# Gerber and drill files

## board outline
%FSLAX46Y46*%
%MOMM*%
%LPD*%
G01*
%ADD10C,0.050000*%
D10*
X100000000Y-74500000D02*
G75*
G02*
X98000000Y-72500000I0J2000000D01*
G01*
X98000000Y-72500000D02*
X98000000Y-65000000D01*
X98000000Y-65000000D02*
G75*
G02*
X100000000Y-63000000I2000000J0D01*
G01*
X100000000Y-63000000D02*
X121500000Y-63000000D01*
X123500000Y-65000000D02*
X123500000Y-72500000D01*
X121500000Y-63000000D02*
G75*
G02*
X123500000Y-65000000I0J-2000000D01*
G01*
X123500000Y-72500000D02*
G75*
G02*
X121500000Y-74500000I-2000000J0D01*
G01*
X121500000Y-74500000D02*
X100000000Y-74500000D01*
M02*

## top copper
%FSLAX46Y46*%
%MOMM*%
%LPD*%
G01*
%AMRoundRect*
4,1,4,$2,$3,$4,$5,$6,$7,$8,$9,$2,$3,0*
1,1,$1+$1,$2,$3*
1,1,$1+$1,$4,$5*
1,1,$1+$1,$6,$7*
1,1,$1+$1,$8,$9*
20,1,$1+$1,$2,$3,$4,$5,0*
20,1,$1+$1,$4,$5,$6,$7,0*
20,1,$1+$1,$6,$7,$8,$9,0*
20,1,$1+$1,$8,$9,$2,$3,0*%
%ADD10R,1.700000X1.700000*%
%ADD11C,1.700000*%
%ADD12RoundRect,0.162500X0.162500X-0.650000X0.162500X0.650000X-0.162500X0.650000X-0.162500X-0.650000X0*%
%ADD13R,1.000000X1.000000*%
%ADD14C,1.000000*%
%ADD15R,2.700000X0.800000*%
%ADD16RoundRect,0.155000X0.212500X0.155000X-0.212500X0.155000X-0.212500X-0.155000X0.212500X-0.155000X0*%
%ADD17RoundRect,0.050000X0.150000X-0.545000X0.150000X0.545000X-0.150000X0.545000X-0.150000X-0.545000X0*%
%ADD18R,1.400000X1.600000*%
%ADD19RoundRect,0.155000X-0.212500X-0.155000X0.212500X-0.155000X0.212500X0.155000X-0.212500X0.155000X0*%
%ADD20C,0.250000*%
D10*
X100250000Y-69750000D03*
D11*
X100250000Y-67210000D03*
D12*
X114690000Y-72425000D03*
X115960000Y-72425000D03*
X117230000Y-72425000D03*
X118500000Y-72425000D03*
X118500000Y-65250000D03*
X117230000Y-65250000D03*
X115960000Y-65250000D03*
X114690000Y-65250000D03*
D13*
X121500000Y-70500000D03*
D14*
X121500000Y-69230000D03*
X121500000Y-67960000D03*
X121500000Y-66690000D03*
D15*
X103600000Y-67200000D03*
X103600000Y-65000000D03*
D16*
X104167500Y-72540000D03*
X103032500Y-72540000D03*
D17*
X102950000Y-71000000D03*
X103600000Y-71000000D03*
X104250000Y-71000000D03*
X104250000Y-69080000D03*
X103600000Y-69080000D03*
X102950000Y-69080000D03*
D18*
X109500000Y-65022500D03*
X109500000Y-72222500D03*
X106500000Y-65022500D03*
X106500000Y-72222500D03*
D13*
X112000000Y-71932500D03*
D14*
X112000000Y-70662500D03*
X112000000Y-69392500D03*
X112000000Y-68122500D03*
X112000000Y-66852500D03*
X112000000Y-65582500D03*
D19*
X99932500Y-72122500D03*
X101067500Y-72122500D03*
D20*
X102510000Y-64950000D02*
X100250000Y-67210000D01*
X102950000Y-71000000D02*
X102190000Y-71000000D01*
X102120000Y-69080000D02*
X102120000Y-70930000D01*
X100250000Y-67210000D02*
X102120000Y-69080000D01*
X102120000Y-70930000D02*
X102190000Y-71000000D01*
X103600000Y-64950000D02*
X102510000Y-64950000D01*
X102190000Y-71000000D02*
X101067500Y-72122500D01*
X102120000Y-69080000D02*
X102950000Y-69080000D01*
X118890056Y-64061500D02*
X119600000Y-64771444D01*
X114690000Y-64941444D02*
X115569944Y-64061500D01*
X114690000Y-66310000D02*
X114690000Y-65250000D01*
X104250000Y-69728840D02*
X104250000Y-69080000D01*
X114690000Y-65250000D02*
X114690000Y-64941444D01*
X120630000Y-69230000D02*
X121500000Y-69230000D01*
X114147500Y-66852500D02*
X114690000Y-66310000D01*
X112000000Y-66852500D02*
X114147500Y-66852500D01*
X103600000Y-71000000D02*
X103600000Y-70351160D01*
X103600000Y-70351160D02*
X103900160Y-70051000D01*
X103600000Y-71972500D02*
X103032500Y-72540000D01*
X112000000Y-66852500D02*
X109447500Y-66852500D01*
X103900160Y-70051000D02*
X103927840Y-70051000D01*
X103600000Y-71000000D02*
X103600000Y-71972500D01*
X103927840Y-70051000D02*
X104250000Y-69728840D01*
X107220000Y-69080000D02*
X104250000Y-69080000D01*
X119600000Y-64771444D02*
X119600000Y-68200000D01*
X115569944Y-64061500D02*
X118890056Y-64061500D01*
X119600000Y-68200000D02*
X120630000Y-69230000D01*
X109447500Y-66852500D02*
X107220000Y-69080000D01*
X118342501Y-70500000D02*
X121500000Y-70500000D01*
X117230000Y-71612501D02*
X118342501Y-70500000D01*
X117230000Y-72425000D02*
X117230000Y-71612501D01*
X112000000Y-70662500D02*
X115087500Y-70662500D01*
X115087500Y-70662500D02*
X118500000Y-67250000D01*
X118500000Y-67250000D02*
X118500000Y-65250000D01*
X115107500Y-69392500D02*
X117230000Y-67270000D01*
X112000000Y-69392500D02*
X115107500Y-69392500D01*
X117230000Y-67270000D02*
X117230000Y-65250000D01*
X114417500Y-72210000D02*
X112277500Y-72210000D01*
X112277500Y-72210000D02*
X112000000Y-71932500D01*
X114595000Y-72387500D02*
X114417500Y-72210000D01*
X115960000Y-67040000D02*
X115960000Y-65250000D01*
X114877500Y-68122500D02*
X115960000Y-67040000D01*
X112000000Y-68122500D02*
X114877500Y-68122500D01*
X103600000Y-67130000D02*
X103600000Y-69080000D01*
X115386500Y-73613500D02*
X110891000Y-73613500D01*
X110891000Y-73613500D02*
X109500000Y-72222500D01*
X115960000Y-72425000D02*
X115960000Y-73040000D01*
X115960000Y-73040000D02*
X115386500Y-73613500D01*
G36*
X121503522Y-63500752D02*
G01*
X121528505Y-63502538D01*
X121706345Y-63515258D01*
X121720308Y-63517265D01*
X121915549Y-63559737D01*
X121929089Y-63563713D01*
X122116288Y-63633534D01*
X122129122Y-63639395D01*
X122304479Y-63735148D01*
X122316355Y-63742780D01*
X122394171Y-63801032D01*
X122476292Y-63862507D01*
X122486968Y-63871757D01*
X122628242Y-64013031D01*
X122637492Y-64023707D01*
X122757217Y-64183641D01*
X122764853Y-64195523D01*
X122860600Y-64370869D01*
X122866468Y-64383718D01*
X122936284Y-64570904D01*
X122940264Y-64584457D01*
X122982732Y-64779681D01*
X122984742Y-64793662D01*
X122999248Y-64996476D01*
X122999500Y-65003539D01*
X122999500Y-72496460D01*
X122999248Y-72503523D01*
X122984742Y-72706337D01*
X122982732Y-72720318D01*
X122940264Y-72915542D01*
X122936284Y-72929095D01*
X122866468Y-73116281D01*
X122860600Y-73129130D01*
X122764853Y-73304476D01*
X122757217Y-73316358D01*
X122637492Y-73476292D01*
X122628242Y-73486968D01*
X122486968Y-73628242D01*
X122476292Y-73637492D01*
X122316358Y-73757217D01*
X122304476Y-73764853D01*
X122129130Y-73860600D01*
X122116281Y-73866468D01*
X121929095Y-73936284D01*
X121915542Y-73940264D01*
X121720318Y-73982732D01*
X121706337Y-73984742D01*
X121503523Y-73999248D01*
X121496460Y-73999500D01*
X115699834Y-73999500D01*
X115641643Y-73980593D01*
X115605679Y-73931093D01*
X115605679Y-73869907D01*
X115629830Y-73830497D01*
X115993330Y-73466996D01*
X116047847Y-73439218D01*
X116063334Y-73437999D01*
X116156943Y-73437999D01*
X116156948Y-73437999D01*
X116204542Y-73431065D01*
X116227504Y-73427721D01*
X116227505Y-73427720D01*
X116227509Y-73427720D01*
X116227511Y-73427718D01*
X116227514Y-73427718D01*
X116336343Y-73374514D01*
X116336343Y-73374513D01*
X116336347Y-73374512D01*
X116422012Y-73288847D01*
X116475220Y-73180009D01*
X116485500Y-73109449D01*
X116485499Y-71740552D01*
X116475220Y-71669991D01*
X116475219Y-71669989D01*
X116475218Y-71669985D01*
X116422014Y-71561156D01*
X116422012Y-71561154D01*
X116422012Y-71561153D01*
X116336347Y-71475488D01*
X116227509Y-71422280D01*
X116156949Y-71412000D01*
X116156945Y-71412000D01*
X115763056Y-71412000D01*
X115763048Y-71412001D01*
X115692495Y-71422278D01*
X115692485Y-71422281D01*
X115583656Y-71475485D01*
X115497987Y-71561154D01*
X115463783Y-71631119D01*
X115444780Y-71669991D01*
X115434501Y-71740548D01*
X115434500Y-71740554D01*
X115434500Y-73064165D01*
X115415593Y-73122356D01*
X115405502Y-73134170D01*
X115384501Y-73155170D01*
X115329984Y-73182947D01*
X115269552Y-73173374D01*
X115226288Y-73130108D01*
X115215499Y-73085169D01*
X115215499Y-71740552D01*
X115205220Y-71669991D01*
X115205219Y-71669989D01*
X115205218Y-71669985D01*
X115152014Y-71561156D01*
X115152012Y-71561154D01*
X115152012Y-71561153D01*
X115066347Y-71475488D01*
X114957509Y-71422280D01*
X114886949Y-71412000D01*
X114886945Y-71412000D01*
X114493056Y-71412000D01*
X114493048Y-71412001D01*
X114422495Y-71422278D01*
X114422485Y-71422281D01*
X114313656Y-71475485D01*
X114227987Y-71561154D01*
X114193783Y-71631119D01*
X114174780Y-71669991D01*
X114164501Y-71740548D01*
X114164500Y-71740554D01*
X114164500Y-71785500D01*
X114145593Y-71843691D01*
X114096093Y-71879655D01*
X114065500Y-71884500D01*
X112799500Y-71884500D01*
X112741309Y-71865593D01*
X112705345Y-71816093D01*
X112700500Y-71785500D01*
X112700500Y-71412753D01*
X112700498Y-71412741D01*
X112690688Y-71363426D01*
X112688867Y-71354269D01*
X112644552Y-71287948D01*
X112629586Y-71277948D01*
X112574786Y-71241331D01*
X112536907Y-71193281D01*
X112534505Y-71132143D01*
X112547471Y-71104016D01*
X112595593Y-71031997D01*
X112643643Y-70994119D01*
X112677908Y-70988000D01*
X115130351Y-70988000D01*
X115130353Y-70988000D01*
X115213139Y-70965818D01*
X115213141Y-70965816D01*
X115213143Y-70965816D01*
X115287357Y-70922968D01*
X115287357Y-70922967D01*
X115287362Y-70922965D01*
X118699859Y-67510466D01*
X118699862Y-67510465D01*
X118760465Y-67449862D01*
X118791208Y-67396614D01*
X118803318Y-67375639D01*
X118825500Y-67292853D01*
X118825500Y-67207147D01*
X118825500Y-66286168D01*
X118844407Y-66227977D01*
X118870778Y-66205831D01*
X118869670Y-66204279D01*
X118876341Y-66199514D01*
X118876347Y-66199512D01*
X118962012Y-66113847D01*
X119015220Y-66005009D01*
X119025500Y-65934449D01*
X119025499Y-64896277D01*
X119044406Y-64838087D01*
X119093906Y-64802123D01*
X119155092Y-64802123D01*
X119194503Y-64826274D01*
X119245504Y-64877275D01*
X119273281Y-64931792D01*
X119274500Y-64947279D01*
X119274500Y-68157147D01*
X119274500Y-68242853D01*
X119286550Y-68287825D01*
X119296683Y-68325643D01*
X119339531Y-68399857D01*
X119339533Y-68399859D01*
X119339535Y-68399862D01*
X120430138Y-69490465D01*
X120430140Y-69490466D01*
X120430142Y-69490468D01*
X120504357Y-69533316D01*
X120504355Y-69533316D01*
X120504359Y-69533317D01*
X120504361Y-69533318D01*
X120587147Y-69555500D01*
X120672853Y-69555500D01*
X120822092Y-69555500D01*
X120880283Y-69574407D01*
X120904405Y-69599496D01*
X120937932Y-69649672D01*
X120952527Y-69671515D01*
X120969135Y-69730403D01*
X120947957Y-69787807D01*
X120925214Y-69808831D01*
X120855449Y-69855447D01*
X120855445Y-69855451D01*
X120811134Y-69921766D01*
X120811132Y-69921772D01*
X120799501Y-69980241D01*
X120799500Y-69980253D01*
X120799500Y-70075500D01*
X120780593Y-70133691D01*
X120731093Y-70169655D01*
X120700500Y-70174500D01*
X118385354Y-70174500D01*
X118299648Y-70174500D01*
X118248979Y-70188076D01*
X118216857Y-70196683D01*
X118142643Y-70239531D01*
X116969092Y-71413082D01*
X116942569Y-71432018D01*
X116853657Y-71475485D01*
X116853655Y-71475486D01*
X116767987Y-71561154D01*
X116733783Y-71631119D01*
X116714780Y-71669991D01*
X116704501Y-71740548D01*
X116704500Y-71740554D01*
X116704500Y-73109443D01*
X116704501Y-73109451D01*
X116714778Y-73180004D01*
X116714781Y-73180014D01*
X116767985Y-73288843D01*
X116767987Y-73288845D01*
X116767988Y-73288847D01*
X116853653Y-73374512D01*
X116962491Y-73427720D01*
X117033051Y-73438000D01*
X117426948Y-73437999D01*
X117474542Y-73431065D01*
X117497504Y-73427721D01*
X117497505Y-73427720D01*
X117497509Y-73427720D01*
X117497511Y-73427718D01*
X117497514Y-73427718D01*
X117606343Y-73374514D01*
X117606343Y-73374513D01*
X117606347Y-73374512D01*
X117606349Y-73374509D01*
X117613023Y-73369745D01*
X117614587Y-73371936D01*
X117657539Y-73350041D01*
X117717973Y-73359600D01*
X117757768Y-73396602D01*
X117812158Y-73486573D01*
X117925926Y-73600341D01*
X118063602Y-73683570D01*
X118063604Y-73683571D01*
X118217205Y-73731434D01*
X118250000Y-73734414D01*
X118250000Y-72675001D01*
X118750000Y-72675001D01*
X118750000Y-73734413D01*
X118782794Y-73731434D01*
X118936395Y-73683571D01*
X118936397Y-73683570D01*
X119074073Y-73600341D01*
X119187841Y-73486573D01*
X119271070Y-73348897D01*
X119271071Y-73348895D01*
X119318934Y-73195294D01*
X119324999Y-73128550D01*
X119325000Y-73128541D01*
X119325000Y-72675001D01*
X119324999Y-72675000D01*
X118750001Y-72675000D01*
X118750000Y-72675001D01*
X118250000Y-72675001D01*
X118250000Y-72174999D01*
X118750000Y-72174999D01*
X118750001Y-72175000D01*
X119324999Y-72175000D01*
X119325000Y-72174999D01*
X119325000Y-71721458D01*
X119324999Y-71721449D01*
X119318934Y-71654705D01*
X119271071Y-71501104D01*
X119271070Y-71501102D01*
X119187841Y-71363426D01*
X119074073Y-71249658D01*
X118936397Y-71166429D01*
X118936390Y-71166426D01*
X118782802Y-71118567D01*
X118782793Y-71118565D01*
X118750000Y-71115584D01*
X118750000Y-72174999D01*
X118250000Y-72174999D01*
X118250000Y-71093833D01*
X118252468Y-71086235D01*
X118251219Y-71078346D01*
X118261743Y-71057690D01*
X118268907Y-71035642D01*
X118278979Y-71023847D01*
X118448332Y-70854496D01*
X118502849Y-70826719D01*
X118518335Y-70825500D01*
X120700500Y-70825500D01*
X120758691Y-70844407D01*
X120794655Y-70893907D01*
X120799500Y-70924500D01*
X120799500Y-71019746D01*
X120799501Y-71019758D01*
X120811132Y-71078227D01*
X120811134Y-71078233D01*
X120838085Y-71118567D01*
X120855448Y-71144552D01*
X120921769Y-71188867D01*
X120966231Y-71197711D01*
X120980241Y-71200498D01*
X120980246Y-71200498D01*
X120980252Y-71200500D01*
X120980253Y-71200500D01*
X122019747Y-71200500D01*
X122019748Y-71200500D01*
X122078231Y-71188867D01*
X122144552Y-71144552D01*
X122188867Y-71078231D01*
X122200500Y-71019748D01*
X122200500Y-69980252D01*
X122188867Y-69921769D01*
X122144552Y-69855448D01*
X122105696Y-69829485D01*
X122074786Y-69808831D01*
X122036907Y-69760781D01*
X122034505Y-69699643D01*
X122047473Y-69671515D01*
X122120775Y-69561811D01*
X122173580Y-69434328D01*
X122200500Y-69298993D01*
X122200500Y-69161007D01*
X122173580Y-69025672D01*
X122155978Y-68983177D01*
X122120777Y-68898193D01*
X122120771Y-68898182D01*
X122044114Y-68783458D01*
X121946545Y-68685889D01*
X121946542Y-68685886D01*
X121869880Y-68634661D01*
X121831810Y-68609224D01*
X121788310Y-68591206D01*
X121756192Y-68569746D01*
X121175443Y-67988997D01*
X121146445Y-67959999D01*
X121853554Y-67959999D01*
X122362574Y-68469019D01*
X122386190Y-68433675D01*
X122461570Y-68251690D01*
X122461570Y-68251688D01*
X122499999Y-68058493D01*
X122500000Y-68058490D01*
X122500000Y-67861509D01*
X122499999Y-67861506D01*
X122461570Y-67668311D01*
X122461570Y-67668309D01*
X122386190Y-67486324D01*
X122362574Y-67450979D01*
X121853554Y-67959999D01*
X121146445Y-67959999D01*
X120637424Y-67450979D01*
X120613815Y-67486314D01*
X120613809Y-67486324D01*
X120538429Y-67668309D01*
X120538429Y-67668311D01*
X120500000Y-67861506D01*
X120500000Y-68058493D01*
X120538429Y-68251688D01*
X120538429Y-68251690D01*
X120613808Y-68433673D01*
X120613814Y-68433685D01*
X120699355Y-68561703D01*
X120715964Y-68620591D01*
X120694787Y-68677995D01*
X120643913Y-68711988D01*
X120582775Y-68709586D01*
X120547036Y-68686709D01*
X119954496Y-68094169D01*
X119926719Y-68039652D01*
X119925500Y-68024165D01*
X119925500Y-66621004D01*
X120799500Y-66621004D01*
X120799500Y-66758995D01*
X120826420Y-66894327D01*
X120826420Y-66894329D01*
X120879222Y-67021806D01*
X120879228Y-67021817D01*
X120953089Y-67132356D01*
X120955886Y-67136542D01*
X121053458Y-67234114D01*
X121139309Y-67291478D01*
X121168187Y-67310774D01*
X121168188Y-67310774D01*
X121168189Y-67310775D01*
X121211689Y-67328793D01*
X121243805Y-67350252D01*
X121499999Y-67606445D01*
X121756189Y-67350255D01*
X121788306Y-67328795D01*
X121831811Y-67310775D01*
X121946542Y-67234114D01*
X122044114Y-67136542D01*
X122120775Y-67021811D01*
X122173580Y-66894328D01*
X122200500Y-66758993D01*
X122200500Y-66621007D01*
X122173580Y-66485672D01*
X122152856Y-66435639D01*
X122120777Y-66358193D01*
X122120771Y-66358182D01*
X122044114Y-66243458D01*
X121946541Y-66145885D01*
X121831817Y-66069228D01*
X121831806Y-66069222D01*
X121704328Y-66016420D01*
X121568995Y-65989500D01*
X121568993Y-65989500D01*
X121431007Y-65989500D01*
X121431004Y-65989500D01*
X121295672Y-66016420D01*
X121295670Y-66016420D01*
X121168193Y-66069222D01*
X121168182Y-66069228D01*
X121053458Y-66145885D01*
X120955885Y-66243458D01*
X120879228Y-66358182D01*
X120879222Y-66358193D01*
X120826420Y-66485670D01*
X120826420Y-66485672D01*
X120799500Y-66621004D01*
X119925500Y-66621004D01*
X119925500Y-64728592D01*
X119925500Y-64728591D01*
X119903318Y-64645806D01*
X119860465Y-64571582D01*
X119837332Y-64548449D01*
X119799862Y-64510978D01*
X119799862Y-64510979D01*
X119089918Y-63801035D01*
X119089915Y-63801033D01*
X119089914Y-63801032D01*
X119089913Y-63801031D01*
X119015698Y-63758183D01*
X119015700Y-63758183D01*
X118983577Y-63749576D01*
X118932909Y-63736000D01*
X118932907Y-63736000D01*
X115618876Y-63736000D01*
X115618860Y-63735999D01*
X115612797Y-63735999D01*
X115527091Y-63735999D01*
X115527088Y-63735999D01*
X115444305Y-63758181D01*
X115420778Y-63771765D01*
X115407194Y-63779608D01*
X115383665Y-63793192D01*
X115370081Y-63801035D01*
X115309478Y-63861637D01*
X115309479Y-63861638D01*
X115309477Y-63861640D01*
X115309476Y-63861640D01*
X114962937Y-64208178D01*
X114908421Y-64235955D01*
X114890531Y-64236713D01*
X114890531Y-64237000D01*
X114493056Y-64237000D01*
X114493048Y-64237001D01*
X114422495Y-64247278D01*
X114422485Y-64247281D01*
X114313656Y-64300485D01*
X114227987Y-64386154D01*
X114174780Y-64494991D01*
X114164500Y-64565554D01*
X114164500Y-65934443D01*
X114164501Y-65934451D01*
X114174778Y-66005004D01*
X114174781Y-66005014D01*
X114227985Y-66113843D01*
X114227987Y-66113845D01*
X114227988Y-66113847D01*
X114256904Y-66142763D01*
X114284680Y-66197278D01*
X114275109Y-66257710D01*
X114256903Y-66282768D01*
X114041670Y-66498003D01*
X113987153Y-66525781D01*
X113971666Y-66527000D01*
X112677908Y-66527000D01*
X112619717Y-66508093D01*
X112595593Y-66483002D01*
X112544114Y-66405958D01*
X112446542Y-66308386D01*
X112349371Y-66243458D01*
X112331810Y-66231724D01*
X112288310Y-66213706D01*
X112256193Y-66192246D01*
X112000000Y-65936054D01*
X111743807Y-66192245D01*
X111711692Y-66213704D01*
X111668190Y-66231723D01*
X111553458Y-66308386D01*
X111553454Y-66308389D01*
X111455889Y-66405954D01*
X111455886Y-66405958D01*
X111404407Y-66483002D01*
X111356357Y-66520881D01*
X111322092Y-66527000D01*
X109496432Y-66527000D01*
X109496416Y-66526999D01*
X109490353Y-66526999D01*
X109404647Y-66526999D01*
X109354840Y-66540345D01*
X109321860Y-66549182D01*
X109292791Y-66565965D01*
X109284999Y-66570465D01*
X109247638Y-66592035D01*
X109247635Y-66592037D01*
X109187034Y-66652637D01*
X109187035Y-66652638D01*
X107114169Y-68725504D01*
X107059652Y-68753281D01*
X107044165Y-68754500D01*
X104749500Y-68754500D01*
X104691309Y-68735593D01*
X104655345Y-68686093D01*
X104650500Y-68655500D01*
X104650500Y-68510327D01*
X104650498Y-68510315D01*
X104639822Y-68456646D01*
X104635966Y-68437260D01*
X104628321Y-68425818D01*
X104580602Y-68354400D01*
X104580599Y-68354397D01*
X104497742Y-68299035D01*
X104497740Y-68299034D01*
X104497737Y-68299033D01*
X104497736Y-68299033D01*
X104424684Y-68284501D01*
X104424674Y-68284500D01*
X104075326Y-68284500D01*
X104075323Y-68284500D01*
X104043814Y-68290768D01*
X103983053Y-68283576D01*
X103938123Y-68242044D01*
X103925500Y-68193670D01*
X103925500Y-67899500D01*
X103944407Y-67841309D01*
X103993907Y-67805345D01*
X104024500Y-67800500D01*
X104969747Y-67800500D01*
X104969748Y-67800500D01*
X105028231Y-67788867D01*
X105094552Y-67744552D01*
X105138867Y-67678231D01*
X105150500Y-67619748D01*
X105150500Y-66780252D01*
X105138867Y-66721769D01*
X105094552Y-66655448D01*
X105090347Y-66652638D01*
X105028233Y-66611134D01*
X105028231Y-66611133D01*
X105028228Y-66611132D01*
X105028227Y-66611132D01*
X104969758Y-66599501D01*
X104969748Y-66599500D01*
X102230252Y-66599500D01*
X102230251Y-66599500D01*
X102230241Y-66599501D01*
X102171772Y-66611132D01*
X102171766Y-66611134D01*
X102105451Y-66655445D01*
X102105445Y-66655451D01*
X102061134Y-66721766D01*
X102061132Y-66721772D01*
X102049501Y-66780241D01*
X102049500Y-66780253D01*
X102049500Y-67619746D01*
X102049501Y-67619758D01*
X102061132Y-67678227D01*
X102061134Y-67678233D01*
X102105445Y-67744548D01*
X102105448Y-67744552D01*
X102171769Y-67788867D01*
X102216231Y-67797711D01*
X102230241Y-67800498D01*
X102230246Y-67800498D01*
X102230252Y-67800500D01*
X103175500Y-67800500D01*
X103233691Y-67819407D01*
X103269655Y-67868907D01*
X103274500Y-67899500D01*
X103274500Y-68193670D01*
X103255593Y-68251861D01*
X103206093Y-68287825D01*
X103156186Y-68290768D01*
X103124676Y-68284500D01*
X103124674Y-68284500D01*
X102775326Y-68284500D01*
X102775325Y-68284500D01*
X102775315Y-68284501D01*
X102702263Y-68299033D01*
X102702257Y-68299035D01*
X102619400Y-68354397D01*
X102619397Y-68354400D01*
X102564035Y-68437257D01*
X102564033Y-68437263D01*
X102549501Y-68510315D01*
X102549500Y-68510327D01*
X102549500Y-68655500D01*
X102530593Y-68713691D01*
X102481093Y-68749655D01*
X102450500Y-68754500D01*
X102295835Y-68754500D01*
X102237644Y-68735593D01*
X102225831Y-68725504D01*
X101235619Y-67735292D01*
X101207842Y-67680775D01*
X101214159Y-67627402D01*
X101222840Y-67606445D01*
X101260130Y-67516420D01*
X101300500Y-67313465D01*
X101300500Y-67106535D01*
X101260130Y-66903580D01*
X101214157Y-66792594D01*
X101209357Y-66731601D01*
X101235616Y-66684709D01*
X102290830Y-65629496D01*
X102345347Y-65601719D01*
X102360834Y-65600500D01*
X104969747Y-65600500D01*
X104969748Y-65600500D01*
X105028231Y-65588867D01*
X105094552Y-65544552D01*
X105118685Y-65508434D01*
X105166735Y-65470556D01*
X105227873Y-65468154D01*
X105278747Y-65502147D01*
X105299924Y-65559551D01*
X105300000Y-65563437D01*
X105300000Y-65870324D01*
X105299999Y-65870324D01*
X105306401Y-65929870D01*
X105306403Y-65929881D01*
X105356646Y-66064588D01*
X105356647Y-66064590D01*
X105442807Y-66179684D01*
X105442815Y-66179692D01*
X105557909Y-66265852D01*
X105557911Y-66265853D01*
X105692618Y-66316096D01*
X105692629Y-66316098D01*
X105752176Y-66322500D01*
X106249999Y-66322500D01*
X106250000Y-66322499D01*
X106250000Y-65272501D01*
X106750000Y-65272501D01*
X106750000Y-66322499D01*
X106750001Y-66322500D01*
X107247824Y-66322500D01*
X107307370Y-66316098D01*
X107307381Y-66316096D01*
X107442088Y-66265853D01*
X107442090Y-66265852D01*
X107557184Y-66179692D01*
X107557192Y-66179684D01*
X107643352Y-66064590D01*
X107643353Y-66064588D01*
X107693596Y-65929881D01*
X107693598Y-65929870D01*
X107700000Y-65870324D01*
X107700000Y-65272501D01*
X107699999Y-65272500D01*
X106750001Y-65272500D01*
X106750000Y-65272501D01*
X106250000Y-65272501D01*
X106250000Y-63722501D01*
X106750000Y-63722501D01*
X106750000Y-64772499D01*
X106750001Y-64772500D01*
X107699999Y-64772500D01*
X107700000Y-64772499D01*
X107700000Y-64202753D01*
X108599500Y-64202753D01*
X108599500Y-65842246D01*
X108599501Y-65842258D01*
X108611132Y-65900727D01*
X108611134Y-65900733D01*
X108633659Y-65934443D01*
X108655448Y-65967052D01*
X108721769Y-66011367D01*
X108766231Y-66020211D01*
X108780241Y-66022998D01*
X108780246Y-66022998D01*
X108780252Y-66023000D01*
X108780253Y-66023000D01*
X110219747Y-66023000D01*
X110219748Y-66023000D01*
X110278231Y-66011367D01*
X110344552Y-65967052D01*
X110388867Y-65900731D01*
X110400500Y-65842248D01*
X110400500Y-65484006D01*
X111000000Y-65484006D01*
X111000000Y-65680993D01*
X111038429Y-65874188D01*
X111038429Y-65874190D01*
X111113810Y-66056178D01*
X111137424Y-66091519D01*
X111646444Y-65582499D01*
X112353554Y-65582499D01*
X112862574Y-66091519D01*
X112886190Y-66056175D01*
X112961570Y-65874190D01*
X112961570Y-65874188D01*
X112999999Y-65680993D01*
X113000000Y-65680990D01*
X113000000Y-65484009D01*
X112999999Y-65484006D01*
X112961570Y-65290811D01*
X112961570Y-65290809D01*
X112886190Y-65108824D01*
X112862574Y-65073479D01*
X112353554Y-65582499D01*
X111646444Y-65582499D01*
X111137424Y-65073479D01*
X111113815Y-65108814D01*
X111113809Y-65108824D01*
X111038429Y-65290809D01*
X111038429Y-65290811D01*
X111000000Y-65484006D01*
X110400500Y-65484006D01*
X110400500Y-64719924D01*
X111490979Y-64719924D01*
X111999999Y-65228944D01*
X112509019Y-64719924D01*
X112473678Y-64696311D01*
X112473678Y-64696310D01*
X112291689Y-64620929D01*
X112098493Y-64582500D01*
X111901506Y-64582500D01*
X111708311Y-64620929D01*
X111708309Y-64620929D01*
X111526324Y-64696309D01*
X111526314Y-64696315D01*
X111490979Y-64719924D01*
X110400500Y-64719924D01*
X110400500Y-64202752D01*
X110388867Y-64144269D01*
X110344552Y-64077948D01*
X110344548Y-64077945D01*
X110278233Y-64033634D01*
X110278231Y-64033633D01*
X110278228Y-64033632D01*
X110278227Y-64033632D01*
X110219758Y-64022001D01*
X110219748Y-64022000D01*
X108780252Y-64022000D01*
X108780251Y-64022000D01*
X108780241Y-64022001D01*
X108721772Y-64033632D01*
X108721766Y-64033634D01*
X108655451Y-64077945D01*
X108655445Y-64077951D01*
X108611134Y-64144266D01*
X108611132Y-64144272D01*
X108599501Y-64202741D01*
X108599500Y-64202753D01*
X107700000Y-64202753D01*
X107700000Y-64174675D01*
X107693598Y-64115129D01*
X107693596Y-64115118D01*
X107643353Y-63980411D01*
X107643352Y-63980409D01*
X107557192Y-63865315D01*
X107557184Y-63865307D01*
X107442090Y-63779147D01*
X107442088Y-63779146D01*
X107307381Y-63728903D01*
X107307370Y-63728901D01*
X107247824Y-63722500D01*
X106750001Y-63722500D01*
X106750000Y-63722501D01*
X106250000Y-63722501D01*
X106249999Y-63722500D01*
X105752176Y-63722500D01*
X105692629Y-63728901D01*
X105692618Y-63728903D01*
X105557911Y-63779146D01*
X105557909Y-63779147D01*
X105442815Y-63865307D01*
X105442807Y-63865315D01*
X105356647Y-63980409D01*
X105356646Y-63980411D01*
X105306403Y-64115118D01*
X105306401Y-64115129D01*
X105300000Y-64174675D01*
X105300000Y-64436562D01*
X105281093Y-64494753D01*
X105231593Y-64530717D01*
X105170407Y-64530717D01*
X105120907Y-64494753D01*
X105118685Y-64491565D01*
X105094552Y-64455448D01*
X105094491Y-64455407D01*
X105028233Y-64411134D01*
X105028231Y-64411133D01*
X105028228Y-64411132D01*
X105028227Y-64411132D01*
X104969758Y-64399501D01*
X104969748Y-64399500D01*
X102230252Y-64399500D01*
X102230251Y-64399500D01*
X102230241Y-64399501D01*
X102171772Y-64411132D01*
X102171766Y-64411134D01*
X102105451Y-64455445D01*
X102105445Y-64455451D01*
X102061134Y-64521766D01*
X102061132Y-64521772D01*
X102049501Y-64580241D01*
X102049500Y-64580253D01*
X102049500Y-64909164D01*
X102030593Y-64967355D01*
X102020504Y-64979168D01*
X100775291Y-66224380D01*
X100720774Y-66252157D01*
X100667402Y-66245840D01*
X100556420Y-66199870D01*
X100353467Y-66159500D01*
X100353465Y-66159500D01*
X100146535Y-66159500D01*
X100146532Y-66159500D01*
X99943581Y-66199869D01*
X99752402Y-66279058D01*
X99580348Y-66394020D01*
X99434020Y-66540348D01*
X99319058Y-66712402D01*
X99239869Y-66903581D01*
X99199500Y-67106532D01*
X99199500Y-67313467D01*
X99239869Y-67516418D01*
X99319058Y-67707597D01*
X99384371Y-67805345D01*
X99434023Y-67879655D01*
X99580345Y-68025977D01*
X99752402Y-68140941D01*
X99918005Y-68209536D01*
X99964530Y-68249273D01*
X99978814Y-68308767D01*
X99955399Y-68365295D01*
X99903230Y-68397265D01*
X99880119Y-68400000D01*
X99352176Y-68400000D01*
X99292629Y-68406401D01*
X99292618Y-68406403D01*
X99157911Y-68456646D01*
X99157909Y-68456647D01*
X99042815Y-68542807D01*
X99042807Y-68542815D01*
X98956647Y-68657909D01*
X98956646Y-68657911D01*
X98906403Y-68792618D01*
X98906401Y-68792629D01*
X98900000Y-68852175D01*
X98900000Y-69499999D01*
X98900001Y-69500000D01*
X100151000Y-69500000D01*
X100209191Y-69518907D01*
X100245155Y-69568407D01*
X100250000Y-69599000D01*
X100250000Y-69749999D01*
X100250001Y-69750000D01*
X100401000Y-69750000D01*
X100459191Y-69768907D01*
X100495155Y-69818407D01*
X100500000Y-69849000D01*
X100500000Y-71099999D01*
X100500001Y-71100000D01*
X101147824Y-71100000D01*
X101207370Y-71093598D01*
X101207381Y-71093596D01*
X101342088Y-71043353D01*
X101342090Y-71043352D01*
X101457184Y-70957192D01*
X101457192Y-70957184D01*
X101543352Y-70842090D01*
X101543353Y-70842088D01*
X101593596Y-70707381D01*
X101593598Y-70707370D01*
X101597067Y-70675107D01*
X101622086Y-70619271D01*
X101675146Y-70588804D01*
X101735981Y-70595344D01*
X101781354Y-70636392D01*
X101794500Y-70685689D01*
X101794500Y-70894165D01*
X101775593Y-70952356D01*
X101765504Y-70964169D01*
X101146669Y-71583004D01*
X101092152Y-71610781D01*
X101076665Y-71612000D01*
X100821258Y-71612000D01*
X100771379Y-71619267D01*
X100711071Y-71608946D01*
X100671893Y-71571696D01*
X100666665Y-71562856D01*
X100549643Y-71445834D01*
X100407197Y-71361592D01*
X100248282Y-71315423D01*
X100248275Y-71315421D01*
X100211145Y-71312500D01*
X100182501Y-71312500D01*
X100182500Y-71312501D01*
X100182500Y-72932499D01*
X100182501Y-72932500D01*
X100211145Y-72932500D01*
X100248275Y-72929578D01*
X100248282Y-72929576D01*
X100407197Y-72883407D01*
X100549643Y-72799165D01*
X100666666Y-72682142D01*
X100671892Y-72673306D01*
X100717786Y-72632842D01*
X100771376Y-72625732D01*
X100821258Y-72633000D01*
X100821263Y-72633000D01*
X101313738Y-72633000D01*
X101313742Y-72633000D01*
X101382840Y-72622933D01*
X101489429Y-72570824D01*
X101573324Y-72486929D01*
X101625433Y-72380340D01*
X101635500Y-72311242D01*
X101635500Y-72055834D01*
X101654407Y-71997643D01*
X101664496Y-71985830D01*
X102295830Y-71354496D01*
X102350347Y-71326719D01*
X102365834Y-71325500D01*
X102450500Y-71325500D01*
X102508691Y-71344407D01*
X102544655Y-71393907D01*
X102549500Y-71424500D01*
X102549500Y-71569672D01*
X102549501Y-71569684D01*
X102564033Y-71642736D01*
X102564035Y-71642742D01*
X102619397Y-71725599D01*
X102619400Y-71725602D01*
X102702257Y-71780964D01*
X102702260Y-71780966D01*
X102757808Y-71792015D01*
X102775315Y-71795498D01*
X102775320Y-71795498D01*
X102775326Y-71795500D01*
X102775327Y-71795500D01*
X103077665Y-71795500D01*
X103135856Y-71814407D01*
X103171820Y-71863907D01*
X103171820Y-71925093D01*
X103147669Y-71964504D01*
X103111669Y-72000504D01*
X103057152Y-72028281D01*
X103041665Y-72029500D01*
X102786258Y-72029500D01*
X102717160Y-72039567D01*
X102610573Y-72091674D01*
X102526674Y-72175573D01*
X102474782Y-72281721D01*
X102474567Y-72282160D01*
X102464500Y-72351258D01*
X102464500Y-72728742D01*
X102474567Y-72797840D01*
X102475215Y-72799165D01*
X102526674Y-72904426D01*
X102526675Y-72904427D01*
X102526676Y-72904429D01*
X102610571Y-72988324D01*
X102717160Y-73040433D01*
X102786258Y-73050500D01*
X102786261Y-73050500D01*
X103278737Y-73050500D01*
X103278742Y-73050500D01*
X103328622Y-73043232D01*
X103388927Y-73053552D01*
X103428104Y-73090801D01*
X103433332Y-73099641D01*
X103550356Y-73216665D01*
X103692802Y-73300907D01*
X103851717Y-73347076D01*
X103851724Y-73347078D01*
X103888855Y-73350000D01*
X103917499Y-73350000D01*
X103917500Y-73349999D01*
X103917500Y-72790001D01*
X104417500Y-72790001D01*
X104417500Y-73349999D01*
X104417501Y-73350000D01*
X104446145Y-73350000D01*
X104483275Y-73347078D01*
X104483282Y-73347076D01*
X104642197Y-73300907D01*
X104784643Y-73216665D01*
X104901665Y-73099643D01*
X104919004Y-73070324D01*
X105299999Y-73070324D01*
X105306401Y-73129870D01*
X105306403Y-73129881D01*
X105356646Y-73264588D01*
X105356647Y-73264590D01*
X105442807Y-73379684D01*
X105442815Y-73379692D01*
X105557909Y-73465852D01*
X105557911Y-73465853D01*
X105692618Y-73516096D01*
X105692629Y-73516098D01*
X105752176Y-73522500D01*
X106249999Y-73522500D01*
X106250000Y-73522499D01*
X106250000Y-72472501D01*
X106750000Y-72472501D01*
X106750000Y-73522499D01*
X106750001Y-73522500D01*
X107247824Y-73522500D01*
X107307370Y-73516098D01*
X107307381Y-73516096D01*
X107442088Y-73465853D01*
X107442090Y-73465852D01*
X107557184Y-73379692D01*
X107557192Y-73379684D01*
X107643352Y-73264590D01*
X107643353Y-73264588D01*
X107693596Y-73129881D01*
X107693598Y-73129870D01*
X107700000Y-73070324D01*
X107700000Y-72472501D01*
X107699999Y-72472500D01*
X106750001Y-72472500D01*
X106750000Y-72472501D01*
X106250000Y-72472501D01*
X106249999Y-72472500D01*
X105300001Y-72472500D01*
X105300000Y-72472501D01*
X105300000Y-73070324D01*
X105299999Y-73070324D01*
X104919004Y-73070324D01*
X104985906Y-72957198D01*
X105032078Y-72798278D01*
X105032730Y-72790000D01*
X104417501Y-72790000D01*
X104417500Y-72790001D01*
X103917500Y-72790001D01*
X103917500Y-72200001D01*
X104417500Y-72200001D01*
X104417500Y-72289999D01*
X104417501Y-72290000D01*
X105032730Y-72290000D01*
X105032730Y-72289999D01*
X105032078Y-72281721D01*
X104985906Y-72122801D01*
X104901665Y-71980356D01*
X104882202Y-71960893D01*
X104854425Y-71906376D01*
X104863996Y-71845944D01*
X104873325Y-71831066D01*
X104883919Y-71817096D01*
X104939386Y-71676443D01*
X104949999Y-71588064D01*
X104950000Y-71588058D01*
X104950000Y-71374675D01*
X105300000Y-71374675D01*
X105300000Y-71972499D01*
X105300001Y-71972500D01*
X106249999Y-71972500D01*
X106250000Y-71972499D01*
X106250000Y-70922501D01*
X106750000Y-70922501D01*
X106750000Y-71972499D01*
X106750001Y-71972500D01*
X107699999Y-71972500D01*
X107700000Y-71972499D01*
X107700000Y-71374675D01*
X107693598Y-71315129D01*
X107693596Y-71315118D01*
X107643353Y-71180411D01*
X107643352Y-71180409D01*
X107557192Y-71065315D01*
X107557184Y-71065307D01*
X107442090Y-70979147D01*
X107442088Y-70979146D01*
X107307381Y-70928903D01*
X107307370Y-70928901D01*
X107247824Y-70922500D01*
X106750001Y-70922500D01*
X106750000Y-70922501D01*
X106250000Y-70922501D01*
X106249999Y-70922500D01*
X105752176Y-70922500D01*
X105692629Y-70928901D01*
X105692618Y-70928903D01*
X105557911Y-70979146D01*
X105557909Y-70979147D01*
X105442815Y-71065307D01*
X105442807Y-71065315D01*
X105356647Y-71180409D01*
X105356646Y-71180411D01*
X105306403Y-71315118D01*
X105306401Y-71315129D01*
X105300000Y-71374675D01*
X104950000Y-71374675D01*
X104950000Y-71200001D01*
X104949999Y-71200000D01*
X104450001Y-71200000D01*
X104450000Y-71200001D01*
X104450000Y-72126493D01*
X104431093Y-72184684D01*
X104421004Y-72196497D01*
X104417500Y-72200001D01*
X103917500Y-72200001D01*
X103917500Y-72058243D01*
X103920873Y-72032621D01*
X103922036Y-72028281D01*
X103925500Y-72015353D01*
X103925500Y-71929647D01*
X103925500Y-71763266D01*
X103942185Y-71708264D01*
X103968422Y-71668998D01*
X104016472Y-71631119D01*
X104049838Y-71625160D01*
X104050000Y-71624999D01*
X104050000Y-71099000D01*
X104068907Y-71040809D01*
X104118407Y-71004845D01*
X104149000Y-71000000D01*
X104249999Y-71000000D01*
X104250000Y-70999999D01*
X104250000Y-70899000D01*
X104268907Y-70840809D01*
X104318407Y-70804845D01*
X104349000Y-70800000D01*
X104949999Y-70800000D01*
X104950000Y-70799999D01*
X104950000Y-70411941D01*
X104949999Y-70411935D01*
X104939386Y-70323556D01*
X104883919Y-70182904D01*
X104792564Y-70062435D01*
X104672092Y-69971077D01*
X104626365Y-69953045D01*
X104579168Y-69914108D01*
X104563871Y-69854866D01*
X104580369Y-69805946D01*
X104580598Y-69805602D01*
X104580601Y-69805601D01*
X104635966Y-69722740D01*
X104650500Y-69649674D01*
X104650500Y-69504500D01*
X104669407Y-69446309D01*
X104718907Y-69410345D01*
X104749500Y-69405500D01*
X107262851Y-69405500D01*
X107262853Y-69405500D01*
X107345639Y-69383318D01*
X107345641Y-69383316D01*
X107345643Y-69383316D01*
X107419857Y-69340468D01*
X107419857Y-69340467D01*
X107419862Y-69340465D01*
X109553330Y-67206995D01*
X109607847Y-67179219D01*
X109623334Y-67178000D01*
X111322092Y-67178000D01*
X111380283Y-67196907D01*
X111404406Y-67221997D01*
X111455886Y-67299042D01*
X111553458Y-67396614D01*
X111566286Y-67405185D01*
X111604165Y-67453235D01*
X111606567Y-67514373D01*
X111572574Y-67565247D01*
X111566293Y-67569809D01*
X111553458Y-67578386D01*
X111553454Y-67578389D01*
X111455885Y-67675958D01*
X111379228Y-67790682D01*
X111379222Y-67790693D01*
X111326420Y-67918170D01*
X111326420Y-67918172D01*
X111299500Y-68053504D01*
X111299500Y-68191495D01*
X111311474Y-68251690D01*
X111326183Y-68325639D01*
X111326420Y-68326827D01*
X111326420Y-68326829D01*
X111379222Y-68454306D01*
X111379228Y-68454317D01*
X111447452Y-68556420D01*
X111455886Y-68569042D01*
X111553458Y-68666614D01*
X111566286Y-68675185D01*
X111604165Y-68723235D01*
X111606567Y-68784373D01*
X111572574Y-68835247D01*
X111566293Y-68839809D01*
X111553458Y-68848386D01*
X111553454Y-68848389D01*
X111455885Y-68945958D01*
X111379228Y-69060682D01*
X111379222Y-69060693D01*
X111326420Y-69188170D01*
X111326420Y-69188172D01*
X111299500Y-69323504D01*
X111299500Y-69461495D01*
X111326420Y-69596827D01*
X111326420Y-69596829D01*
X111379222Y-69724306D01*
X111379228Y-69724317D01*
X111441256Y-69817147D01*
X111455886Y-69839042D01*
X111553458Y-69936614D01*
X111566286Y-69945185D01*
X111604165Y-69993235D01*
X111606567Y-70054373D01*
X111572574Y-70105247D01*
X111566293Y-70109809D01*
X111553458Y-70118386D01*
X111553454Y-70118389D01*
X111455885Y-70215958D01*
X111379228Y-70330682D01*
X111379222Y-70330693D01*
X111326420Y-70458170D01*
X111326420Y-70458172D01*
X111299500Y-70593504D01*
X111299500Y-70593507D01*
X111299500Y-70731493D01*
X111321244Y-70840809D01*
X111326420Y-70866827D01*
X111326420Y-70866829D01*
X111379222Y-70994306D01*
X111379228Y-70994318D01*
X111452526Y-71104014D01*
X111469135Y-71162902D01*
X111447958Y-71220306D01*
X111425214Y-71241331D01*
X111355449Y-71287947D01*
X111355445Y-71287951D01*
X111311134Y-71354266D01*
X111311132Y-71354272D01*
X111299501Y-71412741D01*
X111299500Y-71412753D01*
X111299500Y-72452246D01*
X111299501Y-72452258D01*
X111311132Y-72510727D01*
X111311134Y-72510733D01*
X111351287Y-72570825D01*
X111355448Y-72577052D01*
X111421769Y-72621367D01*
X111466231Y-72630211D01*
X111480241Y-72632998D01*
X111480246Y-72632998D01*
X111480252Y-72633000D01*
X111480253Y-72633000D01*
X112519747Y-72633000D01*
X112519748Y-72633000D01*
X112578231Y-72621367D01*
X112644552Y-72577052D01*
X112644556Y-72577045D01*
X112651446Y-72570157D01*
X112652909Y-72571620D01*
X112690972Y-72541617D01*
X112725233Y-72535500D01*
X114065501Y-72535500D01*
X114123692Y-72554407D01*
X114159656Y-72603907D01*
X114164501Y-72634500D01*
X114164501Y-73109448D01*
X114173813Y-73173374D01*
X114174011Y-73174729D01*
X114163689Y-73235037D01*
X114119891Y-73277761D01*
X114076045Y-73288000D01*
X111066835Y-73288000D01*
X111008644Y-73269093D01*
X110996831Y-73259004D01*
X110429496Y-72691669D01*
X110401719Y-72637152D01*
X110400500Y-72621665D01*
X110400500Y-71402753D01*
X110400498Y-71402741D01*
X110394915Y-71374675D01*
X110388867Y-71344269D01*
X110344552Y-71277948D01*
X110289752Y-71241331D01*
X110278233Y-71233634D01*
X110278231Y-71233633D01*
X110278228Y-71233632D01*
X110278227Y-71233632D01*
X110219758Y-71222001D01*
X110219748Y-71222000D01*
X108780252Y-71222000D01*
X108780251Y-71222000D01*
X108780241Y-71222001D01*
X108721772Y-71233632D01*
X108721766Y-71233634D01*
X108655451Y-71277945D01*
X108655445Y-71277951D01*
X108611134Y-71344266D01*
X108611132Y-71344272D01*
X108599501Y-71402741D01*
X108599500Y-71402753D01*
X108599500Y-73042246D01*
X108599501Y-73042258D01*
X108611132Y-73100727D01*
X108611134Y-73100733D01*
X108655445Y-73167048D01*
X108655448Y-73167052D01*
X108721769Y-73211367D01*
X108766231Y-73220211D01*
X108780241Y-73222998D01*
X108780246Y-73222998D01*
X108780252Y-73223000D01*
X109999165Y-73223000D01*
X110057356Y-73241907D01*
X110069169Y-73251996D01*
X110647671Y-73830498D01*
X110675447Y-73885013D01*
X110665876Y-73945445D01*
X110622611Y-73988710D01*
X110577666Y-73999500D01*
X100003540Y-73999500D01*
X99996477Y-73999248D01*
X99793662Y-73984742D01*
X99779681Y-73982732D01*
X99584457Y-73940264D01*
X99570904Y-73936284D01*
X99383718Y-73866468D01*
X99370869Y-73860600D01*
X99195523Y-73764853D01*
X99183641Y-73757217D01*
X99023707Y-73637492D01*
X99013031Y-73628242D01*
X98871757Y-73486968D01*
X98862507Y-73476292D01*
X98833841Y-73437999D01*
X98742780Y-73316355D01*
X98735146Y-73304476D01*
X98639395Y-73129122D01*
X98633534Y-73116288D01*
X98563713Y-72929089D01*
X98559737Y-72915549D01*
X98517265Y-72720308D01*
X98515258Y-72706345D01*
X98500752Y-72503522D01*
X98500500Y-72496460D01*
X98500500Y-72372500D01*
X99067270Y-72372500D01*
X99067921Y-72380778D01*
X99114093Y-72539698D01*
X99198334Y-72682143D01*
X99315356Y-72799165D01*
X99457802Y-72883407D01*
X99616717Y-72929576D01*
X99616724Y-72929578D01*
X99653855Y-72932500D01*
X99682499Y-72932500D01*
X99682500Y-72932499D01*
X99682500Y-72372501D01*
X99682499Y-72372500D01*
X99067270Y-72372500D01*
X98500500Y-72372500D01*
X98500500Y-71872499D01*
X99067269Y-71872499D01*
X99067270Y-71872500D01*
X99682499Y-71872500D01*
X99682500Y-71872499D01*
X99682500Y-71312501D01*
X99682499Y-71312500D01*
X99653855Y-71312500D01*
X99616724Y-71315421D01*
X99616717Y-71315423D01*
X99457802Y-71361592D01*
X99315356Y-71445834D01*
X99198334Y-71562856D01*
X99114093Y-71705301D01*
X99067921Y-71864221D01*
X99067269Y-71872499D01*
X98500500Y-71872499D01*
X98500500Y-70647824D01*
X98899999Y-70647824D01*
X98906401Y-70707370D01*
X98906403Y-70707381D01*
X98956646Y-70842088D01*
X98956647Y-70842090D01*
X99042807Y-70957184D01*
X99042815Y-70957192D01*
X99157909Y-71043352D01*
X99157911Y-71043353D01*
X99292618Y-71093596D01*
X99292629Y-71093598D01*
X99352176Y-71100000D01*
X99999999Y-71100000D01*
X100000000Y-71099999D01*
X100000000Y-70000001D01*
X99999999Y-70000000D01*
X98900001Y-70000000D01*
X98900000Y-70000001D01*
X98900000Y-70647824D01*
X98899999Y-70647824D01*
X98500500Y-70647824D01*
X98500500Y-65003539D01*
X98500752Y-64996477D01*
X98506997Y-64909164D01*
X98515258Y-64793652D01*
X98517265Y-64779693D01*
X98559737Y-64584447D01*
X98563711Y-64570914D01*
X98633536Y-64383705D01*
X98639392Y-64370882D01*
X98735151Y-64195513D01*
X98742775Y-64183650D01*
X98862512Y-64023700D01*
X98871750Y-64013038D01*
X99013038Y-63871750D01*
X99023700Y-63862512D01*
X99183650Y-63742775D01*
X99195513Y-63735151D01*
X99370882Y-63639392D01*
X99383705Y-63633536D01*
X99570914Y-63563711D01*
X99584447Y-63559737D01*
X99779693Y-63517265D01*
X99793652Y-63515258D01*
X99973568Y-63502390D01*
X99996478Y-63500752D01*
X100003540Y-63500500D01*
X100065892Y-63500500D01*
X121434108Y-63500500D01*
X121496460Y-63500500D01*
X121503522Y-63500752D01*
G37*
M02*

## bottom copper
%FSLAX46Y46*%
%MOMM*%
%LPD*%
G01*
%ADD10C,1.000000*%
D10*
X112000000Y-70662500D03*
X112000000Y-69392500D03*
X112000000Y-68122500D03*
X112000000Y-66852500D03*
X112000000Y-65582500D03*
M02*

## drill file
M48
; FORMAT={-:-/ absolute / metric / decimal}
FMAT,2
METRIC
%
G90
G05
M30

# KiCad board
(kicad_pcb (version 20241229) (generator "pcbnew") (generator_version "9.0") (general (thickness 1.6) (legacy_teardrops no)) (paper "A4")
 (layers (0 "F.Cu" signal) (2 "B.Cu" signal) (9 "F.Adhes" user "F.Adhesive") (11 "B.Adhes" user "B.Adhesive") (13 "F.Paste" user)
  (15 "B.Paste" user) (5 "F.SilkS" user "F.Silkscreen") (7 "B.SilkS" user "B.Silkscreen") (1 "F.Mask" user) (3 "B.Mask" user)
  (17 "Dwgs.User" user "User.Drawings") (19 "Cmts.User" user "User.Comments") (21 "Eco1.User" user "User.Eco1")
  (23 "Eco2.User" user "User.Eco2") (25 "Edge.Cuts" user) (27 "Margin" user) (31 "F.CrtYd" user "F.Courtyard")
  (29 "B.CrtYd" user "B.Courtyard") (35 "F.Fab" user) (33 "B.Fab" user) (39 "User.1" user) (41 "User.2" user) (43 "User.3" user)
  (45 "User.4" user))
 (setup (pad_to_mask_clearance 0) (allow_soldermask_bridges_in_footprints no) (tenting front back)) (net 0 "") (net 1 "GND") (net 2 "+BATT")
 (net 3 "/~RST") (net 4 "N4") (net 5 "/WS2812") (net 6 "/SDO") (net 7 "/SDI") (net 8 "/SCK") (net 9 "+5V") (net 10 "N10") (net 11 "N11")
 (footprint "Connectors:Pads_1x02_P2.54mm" (layer "F.Cu") (at 100.25 69.75 180)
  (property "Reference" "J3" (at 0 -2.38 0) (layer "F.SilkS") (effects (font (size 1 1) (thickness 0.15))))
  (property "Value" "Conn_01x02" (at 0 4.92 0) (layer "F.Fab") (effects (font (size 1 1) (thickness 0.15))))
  (pad "1" smd rect (at 0 0 180) (size 1.7 1.7) (layers "F.Cu" "F.Mask" "F.Paste") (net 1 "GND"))
  (pad "2" smd circle (at 0 2.54 180) (size 1.7 1.7) (layers "F.Cu" "F.Mask" "F.Paste") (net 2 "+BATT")))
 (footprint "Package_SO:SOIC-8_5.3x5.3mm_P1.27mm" (layer "F.Cu") (at 116.595 68.8375 90)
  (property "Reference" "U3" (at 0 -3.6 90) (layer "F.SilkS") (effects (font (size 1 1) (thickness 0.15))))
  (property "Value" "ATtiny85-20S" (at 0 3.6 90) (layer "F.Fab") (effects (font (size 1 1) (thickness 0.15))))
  (pad "1" smd roundrect (at -3.5875 -1.905 90) (size 1.625 0.65) (layers "F.Cu" "F.Mask" "F.Paste") (roundrect_rratio 0.25) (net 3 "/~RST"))
  (pad "2" smd roundrect (at -3.5875 -0.635 90) (size 1.625 0.65) (layers "F.Cu" "F.Mask" "F.Paste") (roundrect_rratio 0.25) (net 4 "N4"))
  (pad "3" smd roundrect (at -3.5875 0.635 90) (size 1.625 0.65) (layers "F.Cu" "F.Mask" "F.Paste") (roundrect_rratio 0.25)
   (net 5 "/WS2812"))
  (pad "4" smd roundrect (at -3.5875 1.905 90) (size 1.625 0.65) (layers "F.Cu" "F.Mask" "F.Paste") (roundrect_rratio 0.25) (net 1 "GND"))
  (pad "5" smd roundrect (at 3.5875 1.905 90) (size 1.625 0.65) (layers "F.Cu" "F.Mask" "F.Paste") (roundrect_rratio 0.25) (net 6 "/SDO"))
  (pad "6" smd roundrect (at 3.5875 0.635 90) (size 1.625 0.65) (layers "F.Cu" "F.Mask" "F.Paste") (roundrect_rratio 0.25) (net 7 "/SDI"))
  (pad "7" smd roundrect (at 3.5875 -0.635 90) (size 1.625 0.65) (layers "F.Cu" "F.Mask" "F.Paste") (roundrect_rratio 0.25) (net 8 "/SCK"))
  (pad "8" smd roundrect (at 3.5875 -1.905 90) (size 1.625 0.65) (layers "F.Cu" "F.Mask" "F.Paste") (roundrect_rratio 0.25) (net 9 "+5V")))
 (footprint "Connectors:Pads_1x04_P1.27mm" (layer "F.Cu") (at 121.5 70.5 180)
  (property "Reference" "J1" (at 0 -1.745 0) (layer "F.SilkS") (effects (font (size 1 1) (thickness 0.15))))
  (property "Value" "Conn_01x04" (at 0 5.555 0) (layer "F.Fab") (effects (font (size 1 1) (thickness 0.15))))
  (pad "1" smd rect (at 0 0 180) (size 1 1) (layers "F.Cu" "F.Mask" "F.Paste") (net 5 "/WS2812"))
  (pad "2" smd circle (at 0 1.27 180) (size 1 1) (layers "F.Cu" "F.Mask" "F.Paste") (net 9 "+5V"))
  (pad "3" smd circle (at 0 2.54 180) (size 1 1) (layers "F.Cu" "F.Mask" "F.Paste") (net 1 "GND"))
  (pad "4" smd circle (at 0 3.81 180) (size 1 1) (layers "F.Cu" "F.Mask" "F.Paste") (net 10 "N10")))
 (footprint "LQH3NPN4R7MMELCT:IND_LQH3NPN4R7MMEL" (layer "F.Cu") (at 103.6 66.1 90)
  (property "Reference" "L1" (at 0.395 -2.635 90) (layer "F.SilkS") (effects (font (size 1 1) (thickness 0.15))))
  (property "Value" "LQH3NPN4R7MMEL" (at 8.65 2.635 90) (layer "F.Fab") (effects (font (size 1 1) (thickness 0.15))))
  (pad "1" smd rect (at -1.1 0 90) (size 0.8 2.7) (layers "F.Cu" "F.Mask" "F.Paste") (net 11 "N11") (solder_mask_margin 0.102))
  (pad "2" smd rect (at 1.1 0 90) (size 0.8 2.7) (layers "F.Cu" "F.Mask" "F.Paste") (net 2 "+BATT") (solder_mask_margin 0.102)))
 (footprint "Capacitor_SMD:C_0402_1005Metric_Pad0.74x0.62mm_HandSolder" (layer "F.Cu") (at 103.6 72.54 180)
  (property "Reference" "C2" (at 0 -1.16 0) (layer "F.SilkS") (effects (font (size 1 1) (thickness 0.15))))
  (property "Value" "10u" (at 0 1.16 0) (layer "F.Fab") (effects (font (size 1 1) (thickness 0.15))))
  (pad "1" smd roundrect (at -0.5675 0 180) (size 0.735 0.62) (layers "F.Cu" "F.Mask" "F.Paste") (roundrect_rratio 0.25) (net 1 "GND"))
  (pad "2" smd roundrect (at 0.5675 0 180) (size 0.735 0.62) (layers "F.Cu" "F.Mask" "F.Paste") (roundrect_rratio 0.25) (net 9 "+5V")))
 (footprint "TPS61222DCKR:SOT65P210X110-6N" (layer "F.Cu") (at 103.6 70.04 90)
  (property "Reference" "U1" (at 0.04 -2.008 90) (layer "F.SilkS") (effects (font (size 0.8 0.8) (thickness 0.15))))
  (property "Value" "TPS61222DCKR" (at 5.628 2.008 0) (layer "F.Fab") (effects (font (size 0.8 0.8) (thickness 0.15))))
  (pad "1" smd roundrect (at -0.96 -0.65 90) (size 1.19 0.4) (layers "F.Cu" "F.Mask" "F.Paste") (roundrect_rratio 0.125) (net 2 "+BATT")
   (solder_mask_margin 0.102))
  (pad "2" smd roundrect (at -0.96 0 90) (size 1.19 0.4) (layers "F.Cu" "F.Mask" "F.Paste") (roundrect_rratio 0.125) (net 9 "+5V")
   (solder_mask_margin 0.102))
  (pad "3" smd roundrect (at -0.96 0.65 90) (size 1.19 0.4) (layers "F.Cu" "F.Mask" "F.Paste") (roundrect_rratio 0.125) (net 1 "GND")
   (solder_mask_margin 0.102))
  (pad "4" smd roundrect (at 0.96 0.65 90) (size 1.19 0.4) (layers "F.Cu" "F.Mask" "F.Paste") (roundrect_rratio 0.125) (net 9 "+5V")
   (solder_mask_margin 0.102))
  (pad "5" smd roundrect (at 0.96 0 90) (size 1.19 0.4) (layers "F.Cu" "F.Mask" "F.Paste") (roundrect_rratio 0.125) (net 11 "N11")
   (solder_mask_margin 0.102))
  (pad "6" smd roundrect (at 0.96 -0.65 90) (size 1.19 0.4) (layers "F.Cu" "F.Mask" "F.Paste") (roundrect_rratio 0.125) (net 2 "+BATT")
   (solder_mask_margin 0.102)))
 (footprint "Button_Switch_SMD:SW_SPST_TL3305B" (layer "F.Cu") (at 108 68.6225 -90)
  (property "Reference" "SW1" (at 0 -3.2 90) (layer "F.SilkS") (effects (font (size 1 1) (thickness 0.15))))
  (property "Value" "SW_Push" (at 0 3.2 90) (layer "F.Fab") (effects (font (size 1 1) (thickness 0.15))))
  (pad "1" smd rect (at -3.6 -1.5 270) (size 1.6 1.4) (layers "F.Cu" "F.Mask" "F.Paste") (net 4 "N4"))
  (pad "1" smd rect (at 3.6 -1.5 270) (size 1.6 1.4) (layers "F.Cu" "F.Mask" "F.Paste") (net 4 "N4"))
  (pad "2" smd rect (at -3.6 1.5 270) (size 1.6 1.4) (layers "F.Cu" "F.Mask" "F.Paste") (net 1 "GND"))
  (pad "2" smd rect (at 3.6 1.5 270) (size 1.6 1.4) (layers "F.Cu" "F.Mask" "F.Paste") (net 1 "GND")))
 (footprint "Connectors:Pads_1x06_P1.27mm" (layer "F.Cu") (at 112 71.9325 180)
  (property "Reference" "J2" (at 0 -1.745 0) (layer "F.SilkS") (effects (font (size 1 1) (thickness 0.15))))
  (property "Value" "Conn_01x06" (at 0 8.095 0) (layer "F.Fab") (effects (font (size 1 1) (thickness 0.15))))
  (pad "1" smd rect (at 0 0 180) (size 1 1) (layers "F.Cu" "F.Mask" "F.Paste") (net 3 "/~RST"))
  (pad "2" smd circle (at 0 1.27 180) (size 1 1) (layers "*.Cu" "*.Mask") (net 6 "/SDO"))
  (pad "3" smd circle (at 0 2.54 180) (size 1 1) (layers "*.Cu" "*.Mask") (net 7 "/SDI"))
  (pad "4" smd circle (at 0 3.81 180) (size 1 1) (layers "*.Cu" "*.Mask") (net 8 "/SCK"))
  (pad "5" smd circle (at 0 5.08 180) (size 1 1) (layers "*.Cu" "*.Mask") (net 9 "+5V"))
  (pad "6" smd circle (at 0 6.35 180) (size 1 1) (layers "*.Cu" "*.Mask") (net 1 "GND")))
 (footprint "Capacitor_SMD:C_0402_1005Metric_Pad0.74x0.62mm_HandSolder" (layer "F.Cu") (at 100.5 72.1225)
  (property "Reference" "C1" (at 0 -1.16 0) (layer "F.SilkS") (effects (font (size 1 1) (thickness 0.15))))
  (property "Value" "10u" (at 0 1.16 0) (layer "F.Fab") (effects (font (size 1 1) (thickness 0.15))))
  (pad "1" smd roundrect (at -0.5675 0) (size 0.735 0.62) (layers "F.Cu" "F.Mask" "F.Paste") (roundrect_rratio 0.25) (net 1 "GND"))
  (pad "2" smd roundrect (at 0.5675 0) (size 0.735 0.62) (layers "F.Cu" "F.Mask" "F.Paste") (roundrect_rratio 0.25) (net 2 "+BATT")))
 (gr_arc (start 100 74.5) (mid 98.585786 73.914214) (end 98 72.5) (stroke (width 0.05) (type default)) (layer "Edge.Cuts"))
 (gr_line (start 98 72.5) (end 98 65) (stroke (width 0.05) (type default)) (layer "Edge.Cuts"))
 (gr_arc (start 98 65) (mid 98.585786 63.585786) (end 100 63) (stroke (width 0.05) (type default)) (layer "Edge.Cuts"))
 (gr_line (start 100 63) (end 121.5 63) (stroke (width 0.05) (type default)) (layer "Edge.Cuts"))
 (gr_line (start 123.5 65) (end 123.5 72.5) (stroke (width 0.05) (type default)) (layer "Edge.Cuts"))
 (gr_arc (start 121.5 63) (mid 122.914214 63.585786) (end 123.5 65) (stroke (width 0.05) (type default)) (layer "Edge.Cuts"))
 (gr_arc (start 123.5 72.5) (mid 122.914214 73.914214) (end 121.5 74.5) (stroke (width 0.05) (type default)) (layer "Edge.Cuts"))
 (gr_line (start 121.5 74.5) (end 100 74.5) (stroke (width 0.05) (type default)) (layer "Edge.Cuts"))
 (segment (start 102.51 64.95) (end 100.25 67.21) (width 0.25) (layer "F.Cu") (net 2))
 (segment (start 102.95 71) (end 102.19 71) (width 0.25) (layer "F.Cu") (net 2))
 (segment (start 102.12 69.08) (end 102.12 70.93) (width 0.25) (layer "F.Cu") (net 2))
 (segment (start 100.25 67.21) (end 102.12 69.08) (width 0.25) (layer "F.Cu") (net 2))
 (segment (start 102.12 70.93) (end 102.19 71) (width 0.25) (layer "F.Cu") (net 2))
 (segment (start 103.6 64.95) (end 102.51 64.95) (width 0.25) (layer "F.Cu") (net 2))
 (segment (start 102.19 71) (end 101.0675 72.1225) (width 0.25) (layer "F.Cu") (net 2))
 (segment (start 102.12 69.08) (end 102.95 69.08) (width 0.25) (layer "F.Cu") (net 2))
 (segment (start 118.890056 64.0615) (end 119.6 64.771444) (width 0.25) (layer "F.Cu") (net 9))
 (segment (start 114.69 64.941444) (end 115.569944 64.0615) (width 0.25) (layer "F.Cu") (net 9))
 (segment (start 114.69 66.31) (end 114.69 65.25) (width 0.25) (layer "F.Cu") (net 9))
 (segment (start 104.25 69.72884) (end 104.25 69.08) (width 0.25) (layer "F.Cu") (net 9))
 (segment (start 114.69 65.25) (end 114.69 64.941444) (width 0.25) (layer "F.Cu") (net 9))
 (segment (start 120.63 69.23) (end 121.5 69.23) (width 0.25) (layer "F.Cu") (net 9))
 (segment (start 114.1475 66.8525) (end 114.69 66.31) (width 0.25) (layer "F.Cu") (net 9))
 (segment (start 112 66.8525) (end 114.1475 66.8525) (width 0.25) (layer "F.Cu") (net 9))
 (segment (start 103.6 71) (end 103.6 70.35116) (width 0.25) (layer "F.Cu") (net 9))
 (segment (start 103.6 70.35116) (end 103.90016 70.051) (width 0.25) (layer "F.Cu") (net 9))
 (segment (start 103.6 71.9725) (end 103.0325 72.54) (width 0.25) (layer "F.Cu") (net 9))
 (segment (start 112 66.8525) (end 109.4475 66.8525) (width 0.25) (layer "F.Cu") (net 9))
 (segment (start 103.90016 70.051) (end 103.92784 70.051) (width 0.25) (layer "F.Cu") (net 9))
 (segment (start 103.6 71) (end 103.6 71.9725) (width 0.25) (layer "F.Cu") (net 9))
 (segment (start 103.92784 70.051) (end 104.25 69.72884) (width 0.25) (layer "F.Cu") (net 9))
 (segment (start 107.22 69.08) (end 104.25 69.08) (width 0.25) (layer "F.Cu") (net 9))
 (segment (start 119.6 64.771444) (end 119.6 68.2) (width 0.25) (layer "F.Cu") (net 9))
 (segment (start 115.569944 64.0615) (end 118.890056 64.0615) (width 0.25) (layer "F.Cu") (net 9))
 (segment (start 119.6 68.2) (end 120.63 69.23) (width 0.25) (layer "F.Cu") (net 9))
 (segment (start 109.4475 66.8525) (end 107.22 69.08) (width 0.25) (layer "F.Cu") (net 9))
 (segment (start 118.342501 70.5) (end 121.5 70.5) (width 0.25) (layer "F.Cu") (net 5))
 (segment (start 117.23 71.612501) (end 118.342501 70.5) (width 0.25) (layer "F.Cu") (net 5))
 (segment (start 117.23 72.425) (end 117.23 71.612501) (width 0.25) (layer "F.Cu") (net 5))
 (segment (start 112 70.6625) (end 115.0875 70.6625) (width 0.25) (layer "F.Cu") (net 6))
 (segment (start 115.0875 70.6625) (end 118.5 67.25) (width 0.25) (layer "F.Cu") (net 6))
 (segment (start 118.5 67.25) (end 118.5 65.25) (width 0.25) (layer "F.Cu") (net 6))
 (segment (start 115.1075 69.3925) (end 117.23 67.27) (width 0.25) (layer "F.Cu") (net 7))
 (segment (start 112 69.3925) (end 115.1075 69.3925) (width 0.25) (layer "F.Cu") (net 7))
 (segment (start 117.23 67.27) (end 117.23 65.25) (width 0.25) (layer "F.Cu") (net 7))
 (segment (start 114.4175 72.21) (end 112.2775 72.21) (width 0.25) (layer "F.Cu") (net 3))
 (segment (start 112.2775 72.21) (end 112 71.9325) (width 0.25) (layer "F.Cu") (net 3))
 (segment (start 114.595 72.3875) (end 114.4175 72.21) (width 0.25) (layer "F.Cu") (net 3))
 (segment (start 115.96 67.04) (end 115.96 65.25) (width 0.25) (layer "F.Cu") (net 8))
 (segment (start 114.8775 68.1225) (end 115.96 67.04) (width 0.25) (layer "F.Cu") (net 8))
 (segment (start 112 68.1225) (end 114.8775 68.1225) (width 0.25) (layer "F.Cu") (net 8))
 (segment (start 103.6 67.13) (end 103.6 69.08) (width 0.25) (layer "F.Cu") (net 11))
 (segment (start 115.3865 73.6135) (end 110.891 73.6135) (width 0.25) (layer "F.Cu") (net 4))
 (segment (start 110.891 73.6135) (end 109.5 72.2225) (width 0.25) (layer "F.Cu") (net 4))
 (segment (start 115.96 72.425) (end 115.96 73.04) (width 0.25) (layer "F.Cu") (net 4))
 (segment (start 115.96 73.04) (end 115.3865 73.6135) (width 0.25) (layer "F.Cu") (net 4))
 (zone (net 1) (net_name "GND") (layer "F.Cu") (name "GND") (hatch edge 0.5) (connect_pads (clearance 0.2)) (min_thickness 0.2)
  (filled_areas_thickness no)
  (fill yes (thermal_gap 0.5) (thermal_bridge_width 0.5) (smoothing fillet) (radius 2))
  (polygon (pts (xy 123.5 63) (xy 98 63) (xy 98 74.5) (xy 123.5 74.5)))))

